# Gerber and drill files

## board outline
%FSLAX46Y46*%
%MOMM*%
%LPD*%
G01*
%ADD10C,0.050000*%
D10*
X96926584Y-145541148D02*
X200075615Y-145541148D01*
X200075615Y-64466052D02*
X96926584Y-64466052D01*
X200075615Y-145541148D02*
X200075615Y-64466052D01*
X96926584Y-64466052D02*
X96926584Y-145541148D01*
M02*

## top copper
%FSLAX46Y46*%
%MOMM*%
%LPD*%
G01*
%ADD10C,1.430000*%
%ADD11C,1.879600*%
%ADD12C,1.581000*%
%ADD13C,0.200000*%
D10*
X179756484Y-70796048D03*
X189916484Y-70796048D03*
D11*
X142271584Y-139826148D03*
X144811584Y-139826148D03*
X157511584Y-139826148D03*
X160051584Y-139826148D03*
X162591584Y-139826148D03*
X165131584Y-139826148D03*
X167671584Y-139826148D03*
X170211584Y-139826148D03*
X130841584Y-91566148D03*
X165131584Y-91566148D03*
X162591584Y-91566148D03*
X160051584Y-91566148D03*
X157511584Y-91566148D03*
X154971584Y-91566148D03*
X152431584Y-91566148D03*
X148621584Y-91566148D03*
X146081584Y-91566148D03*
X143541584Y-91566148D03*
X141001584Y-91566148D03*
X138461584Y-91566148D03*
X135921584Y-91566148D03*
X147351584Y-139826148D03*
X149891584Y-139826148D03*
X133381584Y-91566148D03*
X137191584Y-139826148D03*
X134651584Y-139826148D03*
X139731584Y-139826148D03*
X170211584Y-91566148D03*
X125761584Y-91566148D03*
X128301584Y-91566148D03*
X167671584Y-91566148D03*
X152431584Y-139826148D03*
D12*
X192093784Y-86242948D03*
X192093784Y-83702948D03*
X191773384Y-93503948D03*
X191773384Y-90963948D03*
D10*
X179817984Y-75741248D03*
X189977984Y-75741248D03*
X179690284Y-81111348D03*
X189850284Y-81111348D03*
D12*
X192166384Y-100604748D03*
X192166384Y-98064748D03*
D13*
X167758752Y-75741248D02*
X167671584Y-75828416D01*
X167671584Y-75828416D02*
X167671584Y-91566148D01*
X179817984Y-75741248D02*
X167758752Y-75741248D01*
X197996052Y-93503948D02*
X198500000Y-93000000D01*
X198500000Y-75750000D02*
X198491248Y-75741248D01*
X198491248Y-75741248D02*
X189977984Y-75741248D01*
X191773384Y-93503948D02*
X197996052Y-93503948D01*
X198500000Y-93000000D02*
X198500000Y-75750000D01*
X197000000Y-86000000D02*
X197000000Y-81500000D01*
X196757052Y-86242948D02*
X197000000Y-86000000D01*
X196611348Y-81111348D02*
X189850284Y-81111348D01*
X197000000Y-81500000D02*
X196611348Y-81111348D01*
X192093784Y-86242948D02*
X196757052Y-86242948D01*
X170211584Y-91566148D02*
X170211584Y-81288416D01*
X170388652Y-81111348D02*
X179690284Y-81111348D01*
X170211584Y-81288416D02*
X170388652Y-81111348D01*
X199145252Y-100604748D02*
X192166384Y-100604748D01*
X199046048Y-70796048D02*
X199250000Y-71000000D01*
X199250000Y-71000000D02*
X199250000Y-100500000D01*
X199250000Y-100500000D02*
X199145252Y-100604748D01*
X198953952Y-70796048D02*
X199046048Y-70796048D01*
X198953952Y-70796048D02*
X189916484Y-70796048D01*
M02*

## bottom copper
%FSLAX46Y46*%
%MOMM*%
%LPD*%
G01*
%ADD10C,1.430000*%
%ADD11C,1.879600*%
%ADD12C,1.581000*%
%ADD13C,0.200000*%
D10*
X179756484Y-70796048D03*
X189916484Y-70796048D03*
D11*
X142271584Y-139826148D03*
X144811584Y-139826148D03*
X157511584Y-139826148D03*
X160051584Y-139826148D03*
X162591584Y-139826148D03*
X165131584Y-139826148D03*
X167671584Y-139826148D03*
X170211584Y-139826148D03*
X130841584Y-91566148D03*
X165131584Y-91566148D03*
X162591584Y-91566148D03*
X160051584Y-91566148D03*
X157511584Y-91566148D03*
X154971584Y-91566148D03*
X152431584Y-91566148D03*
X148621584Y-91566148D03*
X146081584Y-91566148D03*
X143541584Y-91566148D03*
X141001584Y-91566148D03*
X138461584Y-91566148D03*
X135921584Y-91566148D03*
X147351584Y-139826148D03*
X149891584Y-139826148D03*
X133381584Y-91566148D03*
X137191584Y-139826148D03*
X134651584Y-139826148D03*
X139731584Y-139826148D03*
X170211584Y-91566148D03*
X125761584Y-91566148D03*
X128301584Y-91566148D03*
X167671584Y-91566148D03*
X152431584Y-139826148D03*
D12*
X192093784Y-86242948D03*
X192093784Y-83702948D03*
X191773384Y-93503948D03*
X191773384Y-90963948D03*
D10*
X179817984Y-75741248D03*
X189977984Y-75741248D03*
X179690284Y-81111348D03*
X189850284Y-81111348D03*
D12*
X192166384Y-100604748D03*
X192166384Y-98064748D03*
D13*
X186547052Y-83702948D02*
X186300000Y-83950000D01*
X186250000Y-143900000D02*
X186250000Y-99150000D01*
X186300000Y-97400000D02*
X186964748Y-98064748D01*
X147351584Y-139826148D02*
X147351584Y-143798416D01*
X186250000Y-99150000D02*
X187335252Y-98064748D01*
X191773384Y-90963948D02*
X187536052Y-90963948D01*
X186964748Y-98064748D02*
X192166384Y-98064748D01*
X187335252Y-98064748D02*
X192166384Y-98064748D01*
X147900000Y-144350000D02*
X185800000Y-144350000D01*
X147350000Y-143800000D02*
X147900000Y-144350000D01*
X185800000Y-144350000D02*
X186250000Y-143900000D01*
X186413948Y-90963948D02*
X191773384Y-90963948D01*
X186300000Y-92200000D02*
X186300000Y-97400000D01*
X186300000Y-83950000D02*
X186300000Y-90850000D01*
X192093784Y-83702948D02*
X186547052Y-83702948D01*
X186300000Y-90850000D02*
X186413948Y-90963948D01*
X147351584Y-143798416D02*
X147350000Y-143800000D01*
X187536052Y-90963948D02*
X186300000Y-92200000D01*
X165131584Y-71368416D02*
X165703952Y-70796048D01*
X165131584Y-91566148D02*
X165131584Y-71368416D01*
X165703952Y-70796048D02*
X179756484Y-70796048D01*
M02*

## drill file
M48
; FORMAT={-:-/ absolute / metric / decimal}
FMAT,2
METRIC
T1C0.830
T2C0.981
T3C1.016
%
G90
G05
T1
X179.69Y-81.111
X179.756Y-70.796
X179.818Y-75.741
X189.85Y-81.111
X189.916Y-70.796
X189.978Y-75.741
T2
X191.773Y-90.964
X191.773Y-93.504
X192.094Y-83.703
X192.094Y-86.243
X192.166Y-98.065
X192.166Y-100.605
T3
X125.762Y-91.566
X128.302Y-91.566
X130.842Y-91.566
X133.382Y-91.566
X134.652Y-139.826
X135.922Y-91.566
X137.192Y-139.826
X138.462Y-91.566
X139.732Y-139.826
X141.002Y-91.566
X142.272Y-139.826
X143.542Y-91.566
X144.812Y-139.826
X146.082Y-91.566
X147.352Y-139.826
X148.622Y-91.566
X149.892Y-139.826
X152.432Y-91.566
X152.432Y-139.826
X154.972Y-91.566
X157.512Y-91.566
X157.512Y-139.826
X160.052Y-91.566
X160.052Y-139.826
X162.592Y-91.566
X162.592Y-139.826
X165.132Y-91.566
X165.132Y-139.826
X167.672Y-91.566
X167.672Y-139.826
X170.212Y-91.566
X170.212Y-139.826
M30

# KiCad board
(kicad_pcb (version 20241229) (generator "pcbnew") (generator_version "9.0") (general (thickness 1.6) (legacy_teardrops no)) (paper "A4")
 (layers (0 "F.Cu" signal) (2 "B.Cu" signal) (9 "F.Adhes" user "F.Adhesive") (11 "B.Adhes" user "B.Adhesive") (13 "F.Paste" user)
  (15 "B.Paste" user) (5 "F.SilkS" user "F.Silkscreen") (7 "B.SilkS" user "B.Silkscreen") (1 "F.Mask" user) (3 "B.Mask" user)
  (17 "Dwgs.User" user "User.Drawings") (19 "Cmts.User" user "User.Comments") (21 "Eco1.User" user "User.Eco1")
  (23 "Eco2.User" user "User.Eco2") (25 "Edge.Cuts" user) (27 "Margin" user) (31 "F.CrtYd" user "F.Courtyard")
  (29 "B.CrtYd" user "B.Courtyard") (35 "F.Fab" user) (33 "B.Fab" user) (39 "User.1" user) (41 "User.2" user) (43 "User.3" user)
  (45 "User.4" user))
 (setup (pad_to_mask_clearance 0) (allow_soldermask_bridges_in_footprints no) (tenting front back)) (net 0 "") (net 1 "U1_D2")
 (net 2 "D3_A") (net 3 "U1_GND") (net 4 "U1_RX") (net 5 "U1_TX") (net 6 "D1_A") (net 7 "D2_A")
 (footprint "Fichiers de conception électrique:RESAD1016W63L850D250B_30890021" (layer "F.Cu") (at 184.836484 70.796048)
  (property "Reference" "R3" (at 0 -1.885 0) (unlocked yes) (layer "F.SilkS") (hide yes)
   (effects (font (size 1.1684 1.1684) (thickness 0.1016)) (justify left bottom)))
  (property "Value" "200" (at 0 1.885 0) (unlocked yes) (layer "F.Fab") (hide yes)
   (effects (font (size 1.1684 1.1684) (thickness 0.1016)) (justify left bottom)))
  (pad "1" thru_hole circle (at -5.08 0) (size 1.43 1.43) (drill 0.83) (layers "*.Cu" "*.Mask") (remove_unused_layers no) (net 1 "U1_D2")
   (solder_mask_margin 0.1016) (thermal_bridge_angle 0))
  (pad "2" thru_hole circle (at 5.08 0) (size 1.43 1.43) (drill 0.83) (layers "*.Cu" "*.Mask") (remove_unused_layers no) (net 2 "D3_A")
   (solder_mask_margin 0.1016) (thermal_bridge_angle 0)))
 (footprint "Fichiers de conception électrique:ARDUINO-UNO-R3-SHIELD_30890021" (layer "F.Cu") (at 144.811584 115.696148 -90)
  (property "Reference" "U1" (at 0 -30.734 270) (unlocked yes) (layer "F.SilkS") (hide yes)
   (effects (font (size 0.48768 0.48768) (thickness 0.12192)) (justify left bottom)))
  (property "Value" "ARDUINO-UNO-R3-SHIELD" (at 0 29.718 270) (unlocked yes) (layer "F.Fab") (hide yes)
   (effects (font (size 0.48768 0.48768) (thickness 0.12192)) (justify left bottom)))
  (pad "3.3V" thru_hole circle (at 24.13 2.54) (size 1.8796 1.8796) (drill 1.016) (layers "*.Cu" "*.Mask") (remove_unused_layers no)
   (solder_mask_margin 0.1016) (thermal_bridge_angle 0))
  (pad "5V" thru_hole circle (at 24.13 0) (size 1.8796 1.8796) (drill 1.016) (layers "*.Cu" "*.Mask") (remove_unused_layers no)
   (solder_mask_margin 0.1016) (thermal_bridge_angle 0))
  (pad "A0" thru_hole circle (at 24.13 -12.7) (size 1.8796 1.8796) (drill 1.016) (layers "*.Cu" "*.Mask") (remove_unused_layers no)
   (solder_mask_margin 0.1016) (thermal_bridge_angle 0))
  (pad "A1" thru_hole circle (at 24.13 -15.24) (size 1.8796 1.8796) (drill 1.016) (layers "*.Cu" "*.Mask") (remove_unused_layers no)
   (solder_mask_margin 0.1016) (thermal_bridge_angle 0))
  (pad "A2" thru_hole circle (at 24.13 -17.78) (size 1.8796 1.8796) (drill 1.016) (layers "*.Cu" "*.Mask") (remove_unused_layers no)
   (solder_mask_margin 0.1016) (thermal_bridge_angle 0))
  (pad "A3" thru_hole circle (at 24.13 -20.32) (size 1.8796 1.8796) (drill 1.016) (layers "*.Cu" "*.Mask") (remove_unused_layers no)
   (solder_mask_margin 0.1016) (thermal_bridge_angle 0))
  (pad "A4" thru_hole circle (at 24.13 -22.86) (size 1.8796 1.8796) (drill 1.016) (layers "*.Cu" "*.Mask") (remove_unused_layers no)
   (solder_mask_margin 0.1016) (thermal_bridge_angle 0))
  (pad "A5" thru_hole circle (at 24.13 -25.4) (size 1.8796 1.8796) (drill 1.016) (layers "*.Cu" "*.Mask") (remove_unused_layers no)
   (solder_mask_margin 0.1016) (thermal_bridge_angle 0))
  (pad "AREF" thru_hole circle (at -24.13 13.97) (size 1.8796 1.8796) (drill 1.016) (layers "*.Cu" "*.Mask") (remove_unused_layers no)
   (solder_mask_margin 0.1016) (thermal_bridge_angle 0))
  (pad "D2" thru_hole circle (at -24.13 -20.32) (size 1.8796 1.8796) (drill 1.016) (layers "*.Cu" "*.Mask") (remove_unused_layers no)
   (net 1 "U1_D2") (solder_mask_margin 0.1016) (thermal_bridge_angle 0))
  (pad "D3" thru_hole circle (at -24.13 -17.78) (size 1.8796 1.8796) (drill 1.016) (layers "*.Cu" "*.Mask") (remove_unused_layers no)
   (solder_mask_margin 0.1016) (thermal_bridge_angle 0))
  (pad "D4" thru_hole circle (at -24.13 -15.24) (size 1.8796 1.8796) (drill 1.016) (layers "*.Cu" "*.Mask") (remove_unused_layers no)
   (solder_mask_margin 0.1016) (thermal_bridge_angle 0))
  (pad "D5" thru_hole circle (at -24.13 -12.7) (size 1.8796 1.8796) (drill 1.016) (layers "*.Cu" "*.Mask") (remove_unused_layers no)
   (solder_mask_margin 0.1016) (thermal_bridge_angle 0))
  (pad "D6" thru_hole circle (at -24.13 -10.16) (size 1.8796 1.8796) (drill 1.016) (layers "*.Cu" "*.Mask") (remove_unused_layers no)
   (solder_mask_margin 0.1016) (thermal_bridge_angle 0))
  (pad "D7" thru_hole circle (at -24.13 -7.62) (size 1.8796 1.8796) (drill 1.016) (layers "*.Cu" "*.Mask") (remove_unused_layers no)
   (solder_mask_margin 0.1016) (thermal_bridge_angle 0))
  (pad "D8" thru_hole circle (at -24.13 -3.81) (size 1.8796 1.8796) (drill 1.016) (layers "*.Cu" "*.Mask") (remove_unused_layers no)
   (solder_mask_margin 0.1016) (thermal_bridge_angle 0))
  (pad "D9" thru_hole circle (at -24.13 -1.27) (size 1.8796 1.8796) (drill 1.016) (layers "*.Cu" "*.Mask") (remove_unused_layers no)
   (solder_mask_margin 0.1016) (thermal_bridge_angle 0))
  (pad "D10" thru_hole circle (at -24.13 1.27) (size 1.8796 1.8796) (drill 1.016) (layers "*.Cu" "*.Mask") (remove_unused_layers no)
   (solder_mask_margin 0.1016) (thermal_bridge_angle 0))
  (pad "D11" thru_hole circle (at -24.13 3.81) (size 1.8796 1.8796) (drill 1.016) (layers "*.Cu" "*.Mask") (remove_unused_layers no)
   (solder_mask_margin 0.1016) (thermal_bridge_angle 0))
  (pad "D12" thru_hole circle (at -24.13 6.35) (size 1.8796 1.8796) (drill 1.016) (layers "*.Cu" "*.Mask") (remove_unused_layers no)
   (solder_mask_margin 0.1016) (thermal_bridge_angle 0))
  (pad "D13" thru_hole circle (at -24.13 8.89) (size 1.8796 1.8796) (drill 1.016) (layers "*.Cu" "*.Mask") (remove_unused_layers no)
   (solder_mask_margin 0.1016) (thermal_bridge_angle 0))
  (pad "GND@0" thru_hole circle (at 24.13 -2.54) (size 1.8796 1.8796) (drill 1.016) (layers "*.Cu" "*.Mask") (remove_unused_layers no)
   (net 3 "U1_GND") (solder_mask_margin 0.1016) (thermal_bridge_angle 0))
  (pad "GND@1" thru_hole circle (at 24.13 -5.08) (size 1.8796 1.8796) (drill 1.016) (layers "*.Cu" "*.Mask") (remove_unused_layers no)
   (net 3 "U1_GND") (solder_mask_margin 0.1016) (thermal_bridge_angle 0))
  (pad "GND@2" thru_hole circle (at -24.13 11.43) (size 1.8796 1.8796) (drill 1.016) (layers "*.Cu" "*.Mask") (remove_unused_layers no)
   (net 3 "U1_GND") (solder_mask_margin 0.1016) (thermal_bridge_angle 0))
  (pad "IOREF" thru_hole circle (at 24.13 7.62) (size 1.8796 1.8796) (drill 1.016) (layers "*.Cu" "*.Mask") (remove_unused_layers no)
   (solder_mask_margin 0.1016) (thermal_bridge_angle 0))
  (pad "NC" thru_hole circle (at 24.13 10.16) (size 1.8796 1.8796) (drill 1.016) (layers "*.Cu" "*.Mask") (remove_unused_layers no)
   (solder_mask_margin 0.1016) (thermal_bridge_angle 0))
  (pad "RES" thru_hole circle (at 24.13 5.08) (size 1.8796 1.8796) (drill 1.016) (layers "*.Cu" "*.Mask") (remove_unused_layers no)
   (solder_mask_margin 0.1016) (thermal_bridge_angle 0))
  (pad "RX" thru_hole circle (at -24.13 -25.4) (size 1.8796 1.8796) (drill 1.016) (layers "*.Cu" "*.Mask") (remove_unused_layers no)
   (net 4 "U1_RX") (solder_mask_margin 0.1016) (thermal_bridge_angle 0))
  (pad "SCL" thru_hole circle (at -24.13 19.05) (size 1.8796 1.8796) (drill 1.016) (layers "*.Cu" "*.Mask") (remove_unused_layers no)
   (solder_mask_margin 0.1016) (thermal_bridge_angle 0))
  (pad "SDA" thru_hole circle (at -24.13 16.51) (size 1.8796 1.8796) (drill 1.016) (layers "*.Cu" "*.Mask") (remove_unused_layers no)
   (solder_mask_margin 0.1016) (thermal_bridge_angle 0))
  (pad "TX" thru_hole circle (at -24.13 -22.86) (size 1.8796 1.8796) (drill 1.016) (layers "*.Cu" "*.Mask") (remove_unused_layers no)
   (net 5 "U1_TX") (solder_mask_margin 0.1016) (thermal_bridge_angle 0))
  (pad "VIN" thru_hole circle (at 24.13 -7.62) (size 1.8796 1.8796) (drill 1.016) (layers "*.Cu" "*.Mask") (remove_unused_layers no)
   (solder_mask_margin 0.1016) (thermal_bridge_angle 0)))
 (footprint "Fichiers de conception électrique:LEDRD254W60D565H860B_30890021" (layer "F.Cu") (at 192.093784 84.972948 90)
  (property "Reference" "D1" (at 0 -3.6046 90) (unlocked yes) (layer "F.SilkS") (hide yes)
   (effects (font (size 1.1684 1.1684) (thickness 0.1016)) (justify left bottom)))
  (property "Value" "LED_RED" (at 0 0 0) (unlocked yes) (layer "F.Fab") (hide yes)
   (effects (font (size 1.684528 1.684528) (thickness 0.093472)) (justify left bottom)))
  (pad "1" thru_hole circle (at -1.27 0 90) (size 1.581 1.581) (drill 0.981) (layers "*.Cu" "*.Mask") (remove_unused_layers no)
   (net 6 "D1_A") (solder_mask_margin 0.1016) (thermal_bridge_angle 0))
  (pad "2" thru_hole circle (at 1.27 0 90) (size 1.581 1.581) (drill 0.981) (layers "*.Cu" "*.Mask") (remove_unused_layers no)
   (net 3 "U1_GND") (solder_mask_margin 0.1016) (thermal_bridge_angle 0)))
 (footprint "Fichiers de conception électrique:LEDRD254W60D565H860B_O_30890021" (layer "F.Cu") (at 191.773384 92.233948 90)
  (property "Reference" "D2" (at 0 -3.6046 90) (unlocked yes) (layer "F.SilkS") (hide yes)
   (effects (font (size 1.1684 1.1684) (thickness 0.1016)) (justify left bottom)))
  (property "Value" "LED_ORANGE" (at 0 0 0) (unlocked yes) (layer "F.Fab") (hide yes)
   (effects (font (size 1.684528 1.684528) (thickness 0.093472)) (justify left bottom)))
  (pad "1" thru_hole circle (at -1.27 0 90) (size 1.581 1.581) (drill 0.981) (layers "*.Cu" "*.Mask") (remove_unused_layers no)
   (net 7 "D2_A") (solder_mask_margin 0.1016) (thermal_bridge_angle 0))
  (pad "2" thru_hole circle (at 1.27 0 90) (size 1.581 1.581) (drill 0.981) (layers "*.Cu" "*.Mask") (remove_unused_layers no)
   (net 3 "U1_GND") (solder_mask_margin 0.1016) (thermal_bridge_angle 0)))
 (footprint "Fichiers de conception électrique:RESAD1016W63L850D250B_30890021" (layer "F.Cu") (at 184.897984 75.741248)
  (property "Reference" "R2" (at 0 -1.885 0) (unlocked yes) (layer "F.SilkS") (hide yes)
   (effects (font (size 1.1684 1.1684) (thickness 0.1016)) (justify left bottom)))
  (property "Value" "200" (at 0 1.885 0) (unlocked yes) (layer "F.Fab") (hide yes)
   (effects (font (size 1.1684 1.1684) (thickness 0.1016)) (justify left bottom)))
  (pad "1" thru_hole circle (at -5.08 0) (size 1.43 1.43) (drill 0.83) (layers "*.Cu" "*.Mask") (remove_unused_layers no) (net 5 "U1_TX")
   (solder_mask_margin 0.1016) (thermal_bridge_angle 0))
  (pad "2" thru_hole circle (at 5.08 0) (size 1.43 1.43) (drill 0.83) (layers "*.Cu" "*.Mask") (remove_unused_layers no) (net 7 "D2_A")
   (solder_mask_margin 0.1016) (thermal_bridge_angle 0)))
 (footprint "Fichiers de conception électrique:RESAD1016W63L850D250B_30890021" (layer "F.Cu") (at 184.770284 81.111348)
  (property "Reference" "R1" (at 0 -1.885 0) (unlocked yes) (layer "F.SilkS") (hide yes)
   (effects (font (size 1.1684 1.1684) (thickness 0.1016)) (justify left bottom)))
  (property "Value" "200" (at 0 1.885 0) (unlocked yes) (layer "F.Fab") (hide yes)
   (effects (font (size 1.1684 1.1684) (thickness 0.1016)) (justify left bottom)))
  (pad "1" thru_hole circle (at -5.08 0) (size 1.43 1.43) (drill 0.83) (layers "*.Cu" "*.Mask") (remove_unused_layers no) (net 4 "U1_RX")
   (solder_mask_margin 0.1016) (thermal_bridge_angle 0))
  (pad "2" thru_hole circle (at 5.08 0) (size 1.43 1.43) (drill 0.83) (layers "*.Cu" "*.Mask") (remove_unused_layers no) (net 6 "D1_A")
   (solder_mask_margin 0.1016) (thermal_bridge_angle 0)))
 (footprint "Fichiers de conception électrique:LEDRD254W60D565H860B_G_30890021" (layer "F.Cu") (at 192.166384 99.334748 90)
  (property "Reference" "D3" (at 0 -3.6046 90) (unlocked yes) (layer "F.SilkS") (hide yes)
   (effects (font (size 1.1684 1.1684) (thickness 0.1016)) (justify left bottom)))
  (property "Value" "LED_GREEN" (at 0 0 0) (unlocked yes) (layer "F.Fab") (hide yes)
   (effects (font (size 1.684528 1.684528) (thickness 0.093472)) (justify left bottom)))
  (pad "1" thru_hole circle (at -1.27 0 90) (size 1.581 1.581) (drill 0.981) (layers "*.Cu" "*.Mask") (remove_unused_layers no)
   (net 2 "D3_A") (solder_mask_margin 0.1016) (thermal_bridge_angle 0))
  (pad "2" thru_hole circle (at 1.27 0 90) (size 1.581 1.581) (drill 0.981) (layers "*.Cu" "*.Mask") (remove_unused_layers no)
   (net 3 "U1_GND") (solder_mask_margin 0.1016) (thermal_bridge_angle 0)))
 (gr_line (start 96.926584 145.541148) (end 200.075615 145.541148) (stroke (width 0.05) (type solid)) (layer "Edge.Cuts"))
 (gr_line (start 200.075615 64.466052) (end 96.926584 64.466052) (stroke (width 0.05) (type solid)) (layer "Edge.Cuts"))
 (gr_line (start 200.075615 145.541148) (end 200.075615 64.466052) (stroke (width 0.05) (type solid)) (layer "Edge.Cuts"))
 (gr_line (start 96.926584 64.466052) (end 96.926584 145.541148) (stroke (width 0.05) (type solid)) (layer "Edge.Cuts"))
 (segment (start 167.758752 75.741248) (end 167.671584 75.828416) (width 0.2) (layer "F.Cu") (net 5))
 (segment (start 167.671584 75.828416) (end 167.671584 91.566148) (width 0.2) (layer "F.Cu") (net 5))
 (segment (start 179.817984 75.741248) (end 167.758752 75.741248) (width 0.2) (layer "F.Cu") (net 5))
 (segment (start 197.996052 93.503948) (end 198.5 93) (width 0.2) (layer "F.Cu") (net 7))
 (segment (start 198.5 75.75) (end 198.491248 75.741248) (width 0.2) (layer "F.Cu") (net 7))
 (segment (start 198.491248 75.741248) (end 189.977984 75.741248) (width 0.2) (layer "F.Cu") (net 7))
 (segment (start 191.773384 93.503948) (end 197.996052 93.503948) (width 0.2) (layer "F.Cu") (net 7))
 (segment (start 198.5 93) (end 198.5 75.75) (width 0.2) (layer "F.Cu") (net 7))
 (segment (start 186.547052 83.702948) (end 186.3 83.95) (width 0.2) (layer "B.Cu") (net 3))
 (segment (start 186.25 143.9) (end 186.25 99.15) (width 0.2) (layer "B.Cu") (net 3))
 (segment (start 186.3 97.4) (end 186.964748 98.064748) (width 0.2) (layer "B.Cu") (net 3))
 (segment (start 147.351584 139.826148) (end 147.351584 143.798416) (width 0.2) (layer "B.Cu") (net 3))
 (segment (start 186.25 99.15) (end 187.335252 98.064748) (width 0.2) (layer "B.Cu") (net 3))
 (segment (start 191.773384 90.963948) (end 187.536052 90.963948) (width 0.2) (layer "B.Cu") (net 3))
 (segment (start 186.964748 98.064748) (end 192.166384 98.064748) (width 0.2) (layer "B.Cu") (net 3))
 (segment (start 187.335252 98.064748) (end 192.166384 98.064748) (width 0.2) (layer "B.Cu") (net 3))
 (segment (start 147.9 144.35) (end 185.8 144.35) (width 0.2) (layer "B.Cu") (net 3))
 (segment (start 147.35 143.8) (end 147.9 144.35) (width 0.2) (layer "B.Cu") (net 3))
 (segment (start 185.8 144.35) (end 186.25 143.9) (width 0.2) (layer "B.Cu") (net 3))
 (segment (start 186.413948 90.963948) (end 191.773384 90.963948) (width 0.2) (layer "B.Cu") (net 3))
 (segment (start 186.3 92.2) (end 186.3 97.4) (width 0.2) (layer "B.Cu") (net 3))
 (segment (start 186.3 83.95) (end 186.3 90.85) (width 0.2) (layer "B.Cu") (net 3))
 (segment (start 192.093784 83.702948) (end 186.547052 83.702948) (width 0.2) (layer "B.Cu") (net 3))
 (segment (start 186.3 90.85) (end 186.413948 90.963948) (width 0.2) (layer "B.Cu") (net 3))
 (segment (start 147.351584 143.798416) (end 147.35 143.8) (width 0.2) (layer "B.Cu") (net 3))
 (segment (start 187.536052 90.963948) (end 186.3 92.2) (width 0.2) (layer "B.Cu") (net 3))
 (segment (start 197 86) (end 197 81.5) (width 0.2) (layer "F.Cu") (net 6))
 (segment (start 196.757052 86.242948) (end 197 86) (width 0.2) (layer "F.Cu") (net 6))
 (segment (start 196.611348 81.111348) (end 189.850284 81.111348) (width 0.2) (layer "F.Cu") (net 6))
 (segment (start 197 81.5) (end 196.611348 81.111348) (width 0.2) (layer "F.Cu") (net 6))
 (segment (start 192.093784 86.242948) (end 196.757052 86.242948) (width 0.2) (layer "F.Cu") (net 6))
 (segment (start 170.211584 91.566148) (end 170.211584 81.288416) (width 0.2) (layer "F.Cu") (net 4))
 (segment (start 170.388652 81.111348) (end 179.690284 81.111348) (width 0.2) (layer "F.Cu") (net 4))
 (segment (start 170.211584 81.288416) (end 170.388652 81.111348) (width 0.2) (layer "F.Cu") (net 4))
 (segment (start 165.131584 71.368416) (end 165.703952 70.796048) (width 0.2) (layer "B.Cu") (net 1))
 (segment (start 165.131584 91.566148) (end 165.131584 71.368416) (width 0.2) (layer "B.Cu") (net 1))
 (segment (start 165.703952 70.796048) (end 179.756484 70.796048) (width 0.2) (layer "B.Cu") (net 1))
 (segment (start 199.145252 100.604748) (end 192.166384 100.604748) (width 0.2) (layer "F.Cu") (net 2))
 (segment (start 199.046048 70.796048) (end 199.25 71) (width 0.2) (layer "F.Cu") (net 2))
 (segment (start 199.25 71) (end 199.25 100.5) (width 0.2) (layer "F.Cu") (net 2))
 (segment (start 199.25 100.5) (end 199.145252 100.604748) (width 0.2) (layer "F.Cu") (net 2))
 (segment (start 198.953952 70.796048) (end 199.046048 70.796048) (width 0.2) (layer "F.Cu") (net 2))
 (segment (start 198.953952 70.796048) (end 189.916484 70.796048) (width 0.2) (layer "F.Cu") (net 2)))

